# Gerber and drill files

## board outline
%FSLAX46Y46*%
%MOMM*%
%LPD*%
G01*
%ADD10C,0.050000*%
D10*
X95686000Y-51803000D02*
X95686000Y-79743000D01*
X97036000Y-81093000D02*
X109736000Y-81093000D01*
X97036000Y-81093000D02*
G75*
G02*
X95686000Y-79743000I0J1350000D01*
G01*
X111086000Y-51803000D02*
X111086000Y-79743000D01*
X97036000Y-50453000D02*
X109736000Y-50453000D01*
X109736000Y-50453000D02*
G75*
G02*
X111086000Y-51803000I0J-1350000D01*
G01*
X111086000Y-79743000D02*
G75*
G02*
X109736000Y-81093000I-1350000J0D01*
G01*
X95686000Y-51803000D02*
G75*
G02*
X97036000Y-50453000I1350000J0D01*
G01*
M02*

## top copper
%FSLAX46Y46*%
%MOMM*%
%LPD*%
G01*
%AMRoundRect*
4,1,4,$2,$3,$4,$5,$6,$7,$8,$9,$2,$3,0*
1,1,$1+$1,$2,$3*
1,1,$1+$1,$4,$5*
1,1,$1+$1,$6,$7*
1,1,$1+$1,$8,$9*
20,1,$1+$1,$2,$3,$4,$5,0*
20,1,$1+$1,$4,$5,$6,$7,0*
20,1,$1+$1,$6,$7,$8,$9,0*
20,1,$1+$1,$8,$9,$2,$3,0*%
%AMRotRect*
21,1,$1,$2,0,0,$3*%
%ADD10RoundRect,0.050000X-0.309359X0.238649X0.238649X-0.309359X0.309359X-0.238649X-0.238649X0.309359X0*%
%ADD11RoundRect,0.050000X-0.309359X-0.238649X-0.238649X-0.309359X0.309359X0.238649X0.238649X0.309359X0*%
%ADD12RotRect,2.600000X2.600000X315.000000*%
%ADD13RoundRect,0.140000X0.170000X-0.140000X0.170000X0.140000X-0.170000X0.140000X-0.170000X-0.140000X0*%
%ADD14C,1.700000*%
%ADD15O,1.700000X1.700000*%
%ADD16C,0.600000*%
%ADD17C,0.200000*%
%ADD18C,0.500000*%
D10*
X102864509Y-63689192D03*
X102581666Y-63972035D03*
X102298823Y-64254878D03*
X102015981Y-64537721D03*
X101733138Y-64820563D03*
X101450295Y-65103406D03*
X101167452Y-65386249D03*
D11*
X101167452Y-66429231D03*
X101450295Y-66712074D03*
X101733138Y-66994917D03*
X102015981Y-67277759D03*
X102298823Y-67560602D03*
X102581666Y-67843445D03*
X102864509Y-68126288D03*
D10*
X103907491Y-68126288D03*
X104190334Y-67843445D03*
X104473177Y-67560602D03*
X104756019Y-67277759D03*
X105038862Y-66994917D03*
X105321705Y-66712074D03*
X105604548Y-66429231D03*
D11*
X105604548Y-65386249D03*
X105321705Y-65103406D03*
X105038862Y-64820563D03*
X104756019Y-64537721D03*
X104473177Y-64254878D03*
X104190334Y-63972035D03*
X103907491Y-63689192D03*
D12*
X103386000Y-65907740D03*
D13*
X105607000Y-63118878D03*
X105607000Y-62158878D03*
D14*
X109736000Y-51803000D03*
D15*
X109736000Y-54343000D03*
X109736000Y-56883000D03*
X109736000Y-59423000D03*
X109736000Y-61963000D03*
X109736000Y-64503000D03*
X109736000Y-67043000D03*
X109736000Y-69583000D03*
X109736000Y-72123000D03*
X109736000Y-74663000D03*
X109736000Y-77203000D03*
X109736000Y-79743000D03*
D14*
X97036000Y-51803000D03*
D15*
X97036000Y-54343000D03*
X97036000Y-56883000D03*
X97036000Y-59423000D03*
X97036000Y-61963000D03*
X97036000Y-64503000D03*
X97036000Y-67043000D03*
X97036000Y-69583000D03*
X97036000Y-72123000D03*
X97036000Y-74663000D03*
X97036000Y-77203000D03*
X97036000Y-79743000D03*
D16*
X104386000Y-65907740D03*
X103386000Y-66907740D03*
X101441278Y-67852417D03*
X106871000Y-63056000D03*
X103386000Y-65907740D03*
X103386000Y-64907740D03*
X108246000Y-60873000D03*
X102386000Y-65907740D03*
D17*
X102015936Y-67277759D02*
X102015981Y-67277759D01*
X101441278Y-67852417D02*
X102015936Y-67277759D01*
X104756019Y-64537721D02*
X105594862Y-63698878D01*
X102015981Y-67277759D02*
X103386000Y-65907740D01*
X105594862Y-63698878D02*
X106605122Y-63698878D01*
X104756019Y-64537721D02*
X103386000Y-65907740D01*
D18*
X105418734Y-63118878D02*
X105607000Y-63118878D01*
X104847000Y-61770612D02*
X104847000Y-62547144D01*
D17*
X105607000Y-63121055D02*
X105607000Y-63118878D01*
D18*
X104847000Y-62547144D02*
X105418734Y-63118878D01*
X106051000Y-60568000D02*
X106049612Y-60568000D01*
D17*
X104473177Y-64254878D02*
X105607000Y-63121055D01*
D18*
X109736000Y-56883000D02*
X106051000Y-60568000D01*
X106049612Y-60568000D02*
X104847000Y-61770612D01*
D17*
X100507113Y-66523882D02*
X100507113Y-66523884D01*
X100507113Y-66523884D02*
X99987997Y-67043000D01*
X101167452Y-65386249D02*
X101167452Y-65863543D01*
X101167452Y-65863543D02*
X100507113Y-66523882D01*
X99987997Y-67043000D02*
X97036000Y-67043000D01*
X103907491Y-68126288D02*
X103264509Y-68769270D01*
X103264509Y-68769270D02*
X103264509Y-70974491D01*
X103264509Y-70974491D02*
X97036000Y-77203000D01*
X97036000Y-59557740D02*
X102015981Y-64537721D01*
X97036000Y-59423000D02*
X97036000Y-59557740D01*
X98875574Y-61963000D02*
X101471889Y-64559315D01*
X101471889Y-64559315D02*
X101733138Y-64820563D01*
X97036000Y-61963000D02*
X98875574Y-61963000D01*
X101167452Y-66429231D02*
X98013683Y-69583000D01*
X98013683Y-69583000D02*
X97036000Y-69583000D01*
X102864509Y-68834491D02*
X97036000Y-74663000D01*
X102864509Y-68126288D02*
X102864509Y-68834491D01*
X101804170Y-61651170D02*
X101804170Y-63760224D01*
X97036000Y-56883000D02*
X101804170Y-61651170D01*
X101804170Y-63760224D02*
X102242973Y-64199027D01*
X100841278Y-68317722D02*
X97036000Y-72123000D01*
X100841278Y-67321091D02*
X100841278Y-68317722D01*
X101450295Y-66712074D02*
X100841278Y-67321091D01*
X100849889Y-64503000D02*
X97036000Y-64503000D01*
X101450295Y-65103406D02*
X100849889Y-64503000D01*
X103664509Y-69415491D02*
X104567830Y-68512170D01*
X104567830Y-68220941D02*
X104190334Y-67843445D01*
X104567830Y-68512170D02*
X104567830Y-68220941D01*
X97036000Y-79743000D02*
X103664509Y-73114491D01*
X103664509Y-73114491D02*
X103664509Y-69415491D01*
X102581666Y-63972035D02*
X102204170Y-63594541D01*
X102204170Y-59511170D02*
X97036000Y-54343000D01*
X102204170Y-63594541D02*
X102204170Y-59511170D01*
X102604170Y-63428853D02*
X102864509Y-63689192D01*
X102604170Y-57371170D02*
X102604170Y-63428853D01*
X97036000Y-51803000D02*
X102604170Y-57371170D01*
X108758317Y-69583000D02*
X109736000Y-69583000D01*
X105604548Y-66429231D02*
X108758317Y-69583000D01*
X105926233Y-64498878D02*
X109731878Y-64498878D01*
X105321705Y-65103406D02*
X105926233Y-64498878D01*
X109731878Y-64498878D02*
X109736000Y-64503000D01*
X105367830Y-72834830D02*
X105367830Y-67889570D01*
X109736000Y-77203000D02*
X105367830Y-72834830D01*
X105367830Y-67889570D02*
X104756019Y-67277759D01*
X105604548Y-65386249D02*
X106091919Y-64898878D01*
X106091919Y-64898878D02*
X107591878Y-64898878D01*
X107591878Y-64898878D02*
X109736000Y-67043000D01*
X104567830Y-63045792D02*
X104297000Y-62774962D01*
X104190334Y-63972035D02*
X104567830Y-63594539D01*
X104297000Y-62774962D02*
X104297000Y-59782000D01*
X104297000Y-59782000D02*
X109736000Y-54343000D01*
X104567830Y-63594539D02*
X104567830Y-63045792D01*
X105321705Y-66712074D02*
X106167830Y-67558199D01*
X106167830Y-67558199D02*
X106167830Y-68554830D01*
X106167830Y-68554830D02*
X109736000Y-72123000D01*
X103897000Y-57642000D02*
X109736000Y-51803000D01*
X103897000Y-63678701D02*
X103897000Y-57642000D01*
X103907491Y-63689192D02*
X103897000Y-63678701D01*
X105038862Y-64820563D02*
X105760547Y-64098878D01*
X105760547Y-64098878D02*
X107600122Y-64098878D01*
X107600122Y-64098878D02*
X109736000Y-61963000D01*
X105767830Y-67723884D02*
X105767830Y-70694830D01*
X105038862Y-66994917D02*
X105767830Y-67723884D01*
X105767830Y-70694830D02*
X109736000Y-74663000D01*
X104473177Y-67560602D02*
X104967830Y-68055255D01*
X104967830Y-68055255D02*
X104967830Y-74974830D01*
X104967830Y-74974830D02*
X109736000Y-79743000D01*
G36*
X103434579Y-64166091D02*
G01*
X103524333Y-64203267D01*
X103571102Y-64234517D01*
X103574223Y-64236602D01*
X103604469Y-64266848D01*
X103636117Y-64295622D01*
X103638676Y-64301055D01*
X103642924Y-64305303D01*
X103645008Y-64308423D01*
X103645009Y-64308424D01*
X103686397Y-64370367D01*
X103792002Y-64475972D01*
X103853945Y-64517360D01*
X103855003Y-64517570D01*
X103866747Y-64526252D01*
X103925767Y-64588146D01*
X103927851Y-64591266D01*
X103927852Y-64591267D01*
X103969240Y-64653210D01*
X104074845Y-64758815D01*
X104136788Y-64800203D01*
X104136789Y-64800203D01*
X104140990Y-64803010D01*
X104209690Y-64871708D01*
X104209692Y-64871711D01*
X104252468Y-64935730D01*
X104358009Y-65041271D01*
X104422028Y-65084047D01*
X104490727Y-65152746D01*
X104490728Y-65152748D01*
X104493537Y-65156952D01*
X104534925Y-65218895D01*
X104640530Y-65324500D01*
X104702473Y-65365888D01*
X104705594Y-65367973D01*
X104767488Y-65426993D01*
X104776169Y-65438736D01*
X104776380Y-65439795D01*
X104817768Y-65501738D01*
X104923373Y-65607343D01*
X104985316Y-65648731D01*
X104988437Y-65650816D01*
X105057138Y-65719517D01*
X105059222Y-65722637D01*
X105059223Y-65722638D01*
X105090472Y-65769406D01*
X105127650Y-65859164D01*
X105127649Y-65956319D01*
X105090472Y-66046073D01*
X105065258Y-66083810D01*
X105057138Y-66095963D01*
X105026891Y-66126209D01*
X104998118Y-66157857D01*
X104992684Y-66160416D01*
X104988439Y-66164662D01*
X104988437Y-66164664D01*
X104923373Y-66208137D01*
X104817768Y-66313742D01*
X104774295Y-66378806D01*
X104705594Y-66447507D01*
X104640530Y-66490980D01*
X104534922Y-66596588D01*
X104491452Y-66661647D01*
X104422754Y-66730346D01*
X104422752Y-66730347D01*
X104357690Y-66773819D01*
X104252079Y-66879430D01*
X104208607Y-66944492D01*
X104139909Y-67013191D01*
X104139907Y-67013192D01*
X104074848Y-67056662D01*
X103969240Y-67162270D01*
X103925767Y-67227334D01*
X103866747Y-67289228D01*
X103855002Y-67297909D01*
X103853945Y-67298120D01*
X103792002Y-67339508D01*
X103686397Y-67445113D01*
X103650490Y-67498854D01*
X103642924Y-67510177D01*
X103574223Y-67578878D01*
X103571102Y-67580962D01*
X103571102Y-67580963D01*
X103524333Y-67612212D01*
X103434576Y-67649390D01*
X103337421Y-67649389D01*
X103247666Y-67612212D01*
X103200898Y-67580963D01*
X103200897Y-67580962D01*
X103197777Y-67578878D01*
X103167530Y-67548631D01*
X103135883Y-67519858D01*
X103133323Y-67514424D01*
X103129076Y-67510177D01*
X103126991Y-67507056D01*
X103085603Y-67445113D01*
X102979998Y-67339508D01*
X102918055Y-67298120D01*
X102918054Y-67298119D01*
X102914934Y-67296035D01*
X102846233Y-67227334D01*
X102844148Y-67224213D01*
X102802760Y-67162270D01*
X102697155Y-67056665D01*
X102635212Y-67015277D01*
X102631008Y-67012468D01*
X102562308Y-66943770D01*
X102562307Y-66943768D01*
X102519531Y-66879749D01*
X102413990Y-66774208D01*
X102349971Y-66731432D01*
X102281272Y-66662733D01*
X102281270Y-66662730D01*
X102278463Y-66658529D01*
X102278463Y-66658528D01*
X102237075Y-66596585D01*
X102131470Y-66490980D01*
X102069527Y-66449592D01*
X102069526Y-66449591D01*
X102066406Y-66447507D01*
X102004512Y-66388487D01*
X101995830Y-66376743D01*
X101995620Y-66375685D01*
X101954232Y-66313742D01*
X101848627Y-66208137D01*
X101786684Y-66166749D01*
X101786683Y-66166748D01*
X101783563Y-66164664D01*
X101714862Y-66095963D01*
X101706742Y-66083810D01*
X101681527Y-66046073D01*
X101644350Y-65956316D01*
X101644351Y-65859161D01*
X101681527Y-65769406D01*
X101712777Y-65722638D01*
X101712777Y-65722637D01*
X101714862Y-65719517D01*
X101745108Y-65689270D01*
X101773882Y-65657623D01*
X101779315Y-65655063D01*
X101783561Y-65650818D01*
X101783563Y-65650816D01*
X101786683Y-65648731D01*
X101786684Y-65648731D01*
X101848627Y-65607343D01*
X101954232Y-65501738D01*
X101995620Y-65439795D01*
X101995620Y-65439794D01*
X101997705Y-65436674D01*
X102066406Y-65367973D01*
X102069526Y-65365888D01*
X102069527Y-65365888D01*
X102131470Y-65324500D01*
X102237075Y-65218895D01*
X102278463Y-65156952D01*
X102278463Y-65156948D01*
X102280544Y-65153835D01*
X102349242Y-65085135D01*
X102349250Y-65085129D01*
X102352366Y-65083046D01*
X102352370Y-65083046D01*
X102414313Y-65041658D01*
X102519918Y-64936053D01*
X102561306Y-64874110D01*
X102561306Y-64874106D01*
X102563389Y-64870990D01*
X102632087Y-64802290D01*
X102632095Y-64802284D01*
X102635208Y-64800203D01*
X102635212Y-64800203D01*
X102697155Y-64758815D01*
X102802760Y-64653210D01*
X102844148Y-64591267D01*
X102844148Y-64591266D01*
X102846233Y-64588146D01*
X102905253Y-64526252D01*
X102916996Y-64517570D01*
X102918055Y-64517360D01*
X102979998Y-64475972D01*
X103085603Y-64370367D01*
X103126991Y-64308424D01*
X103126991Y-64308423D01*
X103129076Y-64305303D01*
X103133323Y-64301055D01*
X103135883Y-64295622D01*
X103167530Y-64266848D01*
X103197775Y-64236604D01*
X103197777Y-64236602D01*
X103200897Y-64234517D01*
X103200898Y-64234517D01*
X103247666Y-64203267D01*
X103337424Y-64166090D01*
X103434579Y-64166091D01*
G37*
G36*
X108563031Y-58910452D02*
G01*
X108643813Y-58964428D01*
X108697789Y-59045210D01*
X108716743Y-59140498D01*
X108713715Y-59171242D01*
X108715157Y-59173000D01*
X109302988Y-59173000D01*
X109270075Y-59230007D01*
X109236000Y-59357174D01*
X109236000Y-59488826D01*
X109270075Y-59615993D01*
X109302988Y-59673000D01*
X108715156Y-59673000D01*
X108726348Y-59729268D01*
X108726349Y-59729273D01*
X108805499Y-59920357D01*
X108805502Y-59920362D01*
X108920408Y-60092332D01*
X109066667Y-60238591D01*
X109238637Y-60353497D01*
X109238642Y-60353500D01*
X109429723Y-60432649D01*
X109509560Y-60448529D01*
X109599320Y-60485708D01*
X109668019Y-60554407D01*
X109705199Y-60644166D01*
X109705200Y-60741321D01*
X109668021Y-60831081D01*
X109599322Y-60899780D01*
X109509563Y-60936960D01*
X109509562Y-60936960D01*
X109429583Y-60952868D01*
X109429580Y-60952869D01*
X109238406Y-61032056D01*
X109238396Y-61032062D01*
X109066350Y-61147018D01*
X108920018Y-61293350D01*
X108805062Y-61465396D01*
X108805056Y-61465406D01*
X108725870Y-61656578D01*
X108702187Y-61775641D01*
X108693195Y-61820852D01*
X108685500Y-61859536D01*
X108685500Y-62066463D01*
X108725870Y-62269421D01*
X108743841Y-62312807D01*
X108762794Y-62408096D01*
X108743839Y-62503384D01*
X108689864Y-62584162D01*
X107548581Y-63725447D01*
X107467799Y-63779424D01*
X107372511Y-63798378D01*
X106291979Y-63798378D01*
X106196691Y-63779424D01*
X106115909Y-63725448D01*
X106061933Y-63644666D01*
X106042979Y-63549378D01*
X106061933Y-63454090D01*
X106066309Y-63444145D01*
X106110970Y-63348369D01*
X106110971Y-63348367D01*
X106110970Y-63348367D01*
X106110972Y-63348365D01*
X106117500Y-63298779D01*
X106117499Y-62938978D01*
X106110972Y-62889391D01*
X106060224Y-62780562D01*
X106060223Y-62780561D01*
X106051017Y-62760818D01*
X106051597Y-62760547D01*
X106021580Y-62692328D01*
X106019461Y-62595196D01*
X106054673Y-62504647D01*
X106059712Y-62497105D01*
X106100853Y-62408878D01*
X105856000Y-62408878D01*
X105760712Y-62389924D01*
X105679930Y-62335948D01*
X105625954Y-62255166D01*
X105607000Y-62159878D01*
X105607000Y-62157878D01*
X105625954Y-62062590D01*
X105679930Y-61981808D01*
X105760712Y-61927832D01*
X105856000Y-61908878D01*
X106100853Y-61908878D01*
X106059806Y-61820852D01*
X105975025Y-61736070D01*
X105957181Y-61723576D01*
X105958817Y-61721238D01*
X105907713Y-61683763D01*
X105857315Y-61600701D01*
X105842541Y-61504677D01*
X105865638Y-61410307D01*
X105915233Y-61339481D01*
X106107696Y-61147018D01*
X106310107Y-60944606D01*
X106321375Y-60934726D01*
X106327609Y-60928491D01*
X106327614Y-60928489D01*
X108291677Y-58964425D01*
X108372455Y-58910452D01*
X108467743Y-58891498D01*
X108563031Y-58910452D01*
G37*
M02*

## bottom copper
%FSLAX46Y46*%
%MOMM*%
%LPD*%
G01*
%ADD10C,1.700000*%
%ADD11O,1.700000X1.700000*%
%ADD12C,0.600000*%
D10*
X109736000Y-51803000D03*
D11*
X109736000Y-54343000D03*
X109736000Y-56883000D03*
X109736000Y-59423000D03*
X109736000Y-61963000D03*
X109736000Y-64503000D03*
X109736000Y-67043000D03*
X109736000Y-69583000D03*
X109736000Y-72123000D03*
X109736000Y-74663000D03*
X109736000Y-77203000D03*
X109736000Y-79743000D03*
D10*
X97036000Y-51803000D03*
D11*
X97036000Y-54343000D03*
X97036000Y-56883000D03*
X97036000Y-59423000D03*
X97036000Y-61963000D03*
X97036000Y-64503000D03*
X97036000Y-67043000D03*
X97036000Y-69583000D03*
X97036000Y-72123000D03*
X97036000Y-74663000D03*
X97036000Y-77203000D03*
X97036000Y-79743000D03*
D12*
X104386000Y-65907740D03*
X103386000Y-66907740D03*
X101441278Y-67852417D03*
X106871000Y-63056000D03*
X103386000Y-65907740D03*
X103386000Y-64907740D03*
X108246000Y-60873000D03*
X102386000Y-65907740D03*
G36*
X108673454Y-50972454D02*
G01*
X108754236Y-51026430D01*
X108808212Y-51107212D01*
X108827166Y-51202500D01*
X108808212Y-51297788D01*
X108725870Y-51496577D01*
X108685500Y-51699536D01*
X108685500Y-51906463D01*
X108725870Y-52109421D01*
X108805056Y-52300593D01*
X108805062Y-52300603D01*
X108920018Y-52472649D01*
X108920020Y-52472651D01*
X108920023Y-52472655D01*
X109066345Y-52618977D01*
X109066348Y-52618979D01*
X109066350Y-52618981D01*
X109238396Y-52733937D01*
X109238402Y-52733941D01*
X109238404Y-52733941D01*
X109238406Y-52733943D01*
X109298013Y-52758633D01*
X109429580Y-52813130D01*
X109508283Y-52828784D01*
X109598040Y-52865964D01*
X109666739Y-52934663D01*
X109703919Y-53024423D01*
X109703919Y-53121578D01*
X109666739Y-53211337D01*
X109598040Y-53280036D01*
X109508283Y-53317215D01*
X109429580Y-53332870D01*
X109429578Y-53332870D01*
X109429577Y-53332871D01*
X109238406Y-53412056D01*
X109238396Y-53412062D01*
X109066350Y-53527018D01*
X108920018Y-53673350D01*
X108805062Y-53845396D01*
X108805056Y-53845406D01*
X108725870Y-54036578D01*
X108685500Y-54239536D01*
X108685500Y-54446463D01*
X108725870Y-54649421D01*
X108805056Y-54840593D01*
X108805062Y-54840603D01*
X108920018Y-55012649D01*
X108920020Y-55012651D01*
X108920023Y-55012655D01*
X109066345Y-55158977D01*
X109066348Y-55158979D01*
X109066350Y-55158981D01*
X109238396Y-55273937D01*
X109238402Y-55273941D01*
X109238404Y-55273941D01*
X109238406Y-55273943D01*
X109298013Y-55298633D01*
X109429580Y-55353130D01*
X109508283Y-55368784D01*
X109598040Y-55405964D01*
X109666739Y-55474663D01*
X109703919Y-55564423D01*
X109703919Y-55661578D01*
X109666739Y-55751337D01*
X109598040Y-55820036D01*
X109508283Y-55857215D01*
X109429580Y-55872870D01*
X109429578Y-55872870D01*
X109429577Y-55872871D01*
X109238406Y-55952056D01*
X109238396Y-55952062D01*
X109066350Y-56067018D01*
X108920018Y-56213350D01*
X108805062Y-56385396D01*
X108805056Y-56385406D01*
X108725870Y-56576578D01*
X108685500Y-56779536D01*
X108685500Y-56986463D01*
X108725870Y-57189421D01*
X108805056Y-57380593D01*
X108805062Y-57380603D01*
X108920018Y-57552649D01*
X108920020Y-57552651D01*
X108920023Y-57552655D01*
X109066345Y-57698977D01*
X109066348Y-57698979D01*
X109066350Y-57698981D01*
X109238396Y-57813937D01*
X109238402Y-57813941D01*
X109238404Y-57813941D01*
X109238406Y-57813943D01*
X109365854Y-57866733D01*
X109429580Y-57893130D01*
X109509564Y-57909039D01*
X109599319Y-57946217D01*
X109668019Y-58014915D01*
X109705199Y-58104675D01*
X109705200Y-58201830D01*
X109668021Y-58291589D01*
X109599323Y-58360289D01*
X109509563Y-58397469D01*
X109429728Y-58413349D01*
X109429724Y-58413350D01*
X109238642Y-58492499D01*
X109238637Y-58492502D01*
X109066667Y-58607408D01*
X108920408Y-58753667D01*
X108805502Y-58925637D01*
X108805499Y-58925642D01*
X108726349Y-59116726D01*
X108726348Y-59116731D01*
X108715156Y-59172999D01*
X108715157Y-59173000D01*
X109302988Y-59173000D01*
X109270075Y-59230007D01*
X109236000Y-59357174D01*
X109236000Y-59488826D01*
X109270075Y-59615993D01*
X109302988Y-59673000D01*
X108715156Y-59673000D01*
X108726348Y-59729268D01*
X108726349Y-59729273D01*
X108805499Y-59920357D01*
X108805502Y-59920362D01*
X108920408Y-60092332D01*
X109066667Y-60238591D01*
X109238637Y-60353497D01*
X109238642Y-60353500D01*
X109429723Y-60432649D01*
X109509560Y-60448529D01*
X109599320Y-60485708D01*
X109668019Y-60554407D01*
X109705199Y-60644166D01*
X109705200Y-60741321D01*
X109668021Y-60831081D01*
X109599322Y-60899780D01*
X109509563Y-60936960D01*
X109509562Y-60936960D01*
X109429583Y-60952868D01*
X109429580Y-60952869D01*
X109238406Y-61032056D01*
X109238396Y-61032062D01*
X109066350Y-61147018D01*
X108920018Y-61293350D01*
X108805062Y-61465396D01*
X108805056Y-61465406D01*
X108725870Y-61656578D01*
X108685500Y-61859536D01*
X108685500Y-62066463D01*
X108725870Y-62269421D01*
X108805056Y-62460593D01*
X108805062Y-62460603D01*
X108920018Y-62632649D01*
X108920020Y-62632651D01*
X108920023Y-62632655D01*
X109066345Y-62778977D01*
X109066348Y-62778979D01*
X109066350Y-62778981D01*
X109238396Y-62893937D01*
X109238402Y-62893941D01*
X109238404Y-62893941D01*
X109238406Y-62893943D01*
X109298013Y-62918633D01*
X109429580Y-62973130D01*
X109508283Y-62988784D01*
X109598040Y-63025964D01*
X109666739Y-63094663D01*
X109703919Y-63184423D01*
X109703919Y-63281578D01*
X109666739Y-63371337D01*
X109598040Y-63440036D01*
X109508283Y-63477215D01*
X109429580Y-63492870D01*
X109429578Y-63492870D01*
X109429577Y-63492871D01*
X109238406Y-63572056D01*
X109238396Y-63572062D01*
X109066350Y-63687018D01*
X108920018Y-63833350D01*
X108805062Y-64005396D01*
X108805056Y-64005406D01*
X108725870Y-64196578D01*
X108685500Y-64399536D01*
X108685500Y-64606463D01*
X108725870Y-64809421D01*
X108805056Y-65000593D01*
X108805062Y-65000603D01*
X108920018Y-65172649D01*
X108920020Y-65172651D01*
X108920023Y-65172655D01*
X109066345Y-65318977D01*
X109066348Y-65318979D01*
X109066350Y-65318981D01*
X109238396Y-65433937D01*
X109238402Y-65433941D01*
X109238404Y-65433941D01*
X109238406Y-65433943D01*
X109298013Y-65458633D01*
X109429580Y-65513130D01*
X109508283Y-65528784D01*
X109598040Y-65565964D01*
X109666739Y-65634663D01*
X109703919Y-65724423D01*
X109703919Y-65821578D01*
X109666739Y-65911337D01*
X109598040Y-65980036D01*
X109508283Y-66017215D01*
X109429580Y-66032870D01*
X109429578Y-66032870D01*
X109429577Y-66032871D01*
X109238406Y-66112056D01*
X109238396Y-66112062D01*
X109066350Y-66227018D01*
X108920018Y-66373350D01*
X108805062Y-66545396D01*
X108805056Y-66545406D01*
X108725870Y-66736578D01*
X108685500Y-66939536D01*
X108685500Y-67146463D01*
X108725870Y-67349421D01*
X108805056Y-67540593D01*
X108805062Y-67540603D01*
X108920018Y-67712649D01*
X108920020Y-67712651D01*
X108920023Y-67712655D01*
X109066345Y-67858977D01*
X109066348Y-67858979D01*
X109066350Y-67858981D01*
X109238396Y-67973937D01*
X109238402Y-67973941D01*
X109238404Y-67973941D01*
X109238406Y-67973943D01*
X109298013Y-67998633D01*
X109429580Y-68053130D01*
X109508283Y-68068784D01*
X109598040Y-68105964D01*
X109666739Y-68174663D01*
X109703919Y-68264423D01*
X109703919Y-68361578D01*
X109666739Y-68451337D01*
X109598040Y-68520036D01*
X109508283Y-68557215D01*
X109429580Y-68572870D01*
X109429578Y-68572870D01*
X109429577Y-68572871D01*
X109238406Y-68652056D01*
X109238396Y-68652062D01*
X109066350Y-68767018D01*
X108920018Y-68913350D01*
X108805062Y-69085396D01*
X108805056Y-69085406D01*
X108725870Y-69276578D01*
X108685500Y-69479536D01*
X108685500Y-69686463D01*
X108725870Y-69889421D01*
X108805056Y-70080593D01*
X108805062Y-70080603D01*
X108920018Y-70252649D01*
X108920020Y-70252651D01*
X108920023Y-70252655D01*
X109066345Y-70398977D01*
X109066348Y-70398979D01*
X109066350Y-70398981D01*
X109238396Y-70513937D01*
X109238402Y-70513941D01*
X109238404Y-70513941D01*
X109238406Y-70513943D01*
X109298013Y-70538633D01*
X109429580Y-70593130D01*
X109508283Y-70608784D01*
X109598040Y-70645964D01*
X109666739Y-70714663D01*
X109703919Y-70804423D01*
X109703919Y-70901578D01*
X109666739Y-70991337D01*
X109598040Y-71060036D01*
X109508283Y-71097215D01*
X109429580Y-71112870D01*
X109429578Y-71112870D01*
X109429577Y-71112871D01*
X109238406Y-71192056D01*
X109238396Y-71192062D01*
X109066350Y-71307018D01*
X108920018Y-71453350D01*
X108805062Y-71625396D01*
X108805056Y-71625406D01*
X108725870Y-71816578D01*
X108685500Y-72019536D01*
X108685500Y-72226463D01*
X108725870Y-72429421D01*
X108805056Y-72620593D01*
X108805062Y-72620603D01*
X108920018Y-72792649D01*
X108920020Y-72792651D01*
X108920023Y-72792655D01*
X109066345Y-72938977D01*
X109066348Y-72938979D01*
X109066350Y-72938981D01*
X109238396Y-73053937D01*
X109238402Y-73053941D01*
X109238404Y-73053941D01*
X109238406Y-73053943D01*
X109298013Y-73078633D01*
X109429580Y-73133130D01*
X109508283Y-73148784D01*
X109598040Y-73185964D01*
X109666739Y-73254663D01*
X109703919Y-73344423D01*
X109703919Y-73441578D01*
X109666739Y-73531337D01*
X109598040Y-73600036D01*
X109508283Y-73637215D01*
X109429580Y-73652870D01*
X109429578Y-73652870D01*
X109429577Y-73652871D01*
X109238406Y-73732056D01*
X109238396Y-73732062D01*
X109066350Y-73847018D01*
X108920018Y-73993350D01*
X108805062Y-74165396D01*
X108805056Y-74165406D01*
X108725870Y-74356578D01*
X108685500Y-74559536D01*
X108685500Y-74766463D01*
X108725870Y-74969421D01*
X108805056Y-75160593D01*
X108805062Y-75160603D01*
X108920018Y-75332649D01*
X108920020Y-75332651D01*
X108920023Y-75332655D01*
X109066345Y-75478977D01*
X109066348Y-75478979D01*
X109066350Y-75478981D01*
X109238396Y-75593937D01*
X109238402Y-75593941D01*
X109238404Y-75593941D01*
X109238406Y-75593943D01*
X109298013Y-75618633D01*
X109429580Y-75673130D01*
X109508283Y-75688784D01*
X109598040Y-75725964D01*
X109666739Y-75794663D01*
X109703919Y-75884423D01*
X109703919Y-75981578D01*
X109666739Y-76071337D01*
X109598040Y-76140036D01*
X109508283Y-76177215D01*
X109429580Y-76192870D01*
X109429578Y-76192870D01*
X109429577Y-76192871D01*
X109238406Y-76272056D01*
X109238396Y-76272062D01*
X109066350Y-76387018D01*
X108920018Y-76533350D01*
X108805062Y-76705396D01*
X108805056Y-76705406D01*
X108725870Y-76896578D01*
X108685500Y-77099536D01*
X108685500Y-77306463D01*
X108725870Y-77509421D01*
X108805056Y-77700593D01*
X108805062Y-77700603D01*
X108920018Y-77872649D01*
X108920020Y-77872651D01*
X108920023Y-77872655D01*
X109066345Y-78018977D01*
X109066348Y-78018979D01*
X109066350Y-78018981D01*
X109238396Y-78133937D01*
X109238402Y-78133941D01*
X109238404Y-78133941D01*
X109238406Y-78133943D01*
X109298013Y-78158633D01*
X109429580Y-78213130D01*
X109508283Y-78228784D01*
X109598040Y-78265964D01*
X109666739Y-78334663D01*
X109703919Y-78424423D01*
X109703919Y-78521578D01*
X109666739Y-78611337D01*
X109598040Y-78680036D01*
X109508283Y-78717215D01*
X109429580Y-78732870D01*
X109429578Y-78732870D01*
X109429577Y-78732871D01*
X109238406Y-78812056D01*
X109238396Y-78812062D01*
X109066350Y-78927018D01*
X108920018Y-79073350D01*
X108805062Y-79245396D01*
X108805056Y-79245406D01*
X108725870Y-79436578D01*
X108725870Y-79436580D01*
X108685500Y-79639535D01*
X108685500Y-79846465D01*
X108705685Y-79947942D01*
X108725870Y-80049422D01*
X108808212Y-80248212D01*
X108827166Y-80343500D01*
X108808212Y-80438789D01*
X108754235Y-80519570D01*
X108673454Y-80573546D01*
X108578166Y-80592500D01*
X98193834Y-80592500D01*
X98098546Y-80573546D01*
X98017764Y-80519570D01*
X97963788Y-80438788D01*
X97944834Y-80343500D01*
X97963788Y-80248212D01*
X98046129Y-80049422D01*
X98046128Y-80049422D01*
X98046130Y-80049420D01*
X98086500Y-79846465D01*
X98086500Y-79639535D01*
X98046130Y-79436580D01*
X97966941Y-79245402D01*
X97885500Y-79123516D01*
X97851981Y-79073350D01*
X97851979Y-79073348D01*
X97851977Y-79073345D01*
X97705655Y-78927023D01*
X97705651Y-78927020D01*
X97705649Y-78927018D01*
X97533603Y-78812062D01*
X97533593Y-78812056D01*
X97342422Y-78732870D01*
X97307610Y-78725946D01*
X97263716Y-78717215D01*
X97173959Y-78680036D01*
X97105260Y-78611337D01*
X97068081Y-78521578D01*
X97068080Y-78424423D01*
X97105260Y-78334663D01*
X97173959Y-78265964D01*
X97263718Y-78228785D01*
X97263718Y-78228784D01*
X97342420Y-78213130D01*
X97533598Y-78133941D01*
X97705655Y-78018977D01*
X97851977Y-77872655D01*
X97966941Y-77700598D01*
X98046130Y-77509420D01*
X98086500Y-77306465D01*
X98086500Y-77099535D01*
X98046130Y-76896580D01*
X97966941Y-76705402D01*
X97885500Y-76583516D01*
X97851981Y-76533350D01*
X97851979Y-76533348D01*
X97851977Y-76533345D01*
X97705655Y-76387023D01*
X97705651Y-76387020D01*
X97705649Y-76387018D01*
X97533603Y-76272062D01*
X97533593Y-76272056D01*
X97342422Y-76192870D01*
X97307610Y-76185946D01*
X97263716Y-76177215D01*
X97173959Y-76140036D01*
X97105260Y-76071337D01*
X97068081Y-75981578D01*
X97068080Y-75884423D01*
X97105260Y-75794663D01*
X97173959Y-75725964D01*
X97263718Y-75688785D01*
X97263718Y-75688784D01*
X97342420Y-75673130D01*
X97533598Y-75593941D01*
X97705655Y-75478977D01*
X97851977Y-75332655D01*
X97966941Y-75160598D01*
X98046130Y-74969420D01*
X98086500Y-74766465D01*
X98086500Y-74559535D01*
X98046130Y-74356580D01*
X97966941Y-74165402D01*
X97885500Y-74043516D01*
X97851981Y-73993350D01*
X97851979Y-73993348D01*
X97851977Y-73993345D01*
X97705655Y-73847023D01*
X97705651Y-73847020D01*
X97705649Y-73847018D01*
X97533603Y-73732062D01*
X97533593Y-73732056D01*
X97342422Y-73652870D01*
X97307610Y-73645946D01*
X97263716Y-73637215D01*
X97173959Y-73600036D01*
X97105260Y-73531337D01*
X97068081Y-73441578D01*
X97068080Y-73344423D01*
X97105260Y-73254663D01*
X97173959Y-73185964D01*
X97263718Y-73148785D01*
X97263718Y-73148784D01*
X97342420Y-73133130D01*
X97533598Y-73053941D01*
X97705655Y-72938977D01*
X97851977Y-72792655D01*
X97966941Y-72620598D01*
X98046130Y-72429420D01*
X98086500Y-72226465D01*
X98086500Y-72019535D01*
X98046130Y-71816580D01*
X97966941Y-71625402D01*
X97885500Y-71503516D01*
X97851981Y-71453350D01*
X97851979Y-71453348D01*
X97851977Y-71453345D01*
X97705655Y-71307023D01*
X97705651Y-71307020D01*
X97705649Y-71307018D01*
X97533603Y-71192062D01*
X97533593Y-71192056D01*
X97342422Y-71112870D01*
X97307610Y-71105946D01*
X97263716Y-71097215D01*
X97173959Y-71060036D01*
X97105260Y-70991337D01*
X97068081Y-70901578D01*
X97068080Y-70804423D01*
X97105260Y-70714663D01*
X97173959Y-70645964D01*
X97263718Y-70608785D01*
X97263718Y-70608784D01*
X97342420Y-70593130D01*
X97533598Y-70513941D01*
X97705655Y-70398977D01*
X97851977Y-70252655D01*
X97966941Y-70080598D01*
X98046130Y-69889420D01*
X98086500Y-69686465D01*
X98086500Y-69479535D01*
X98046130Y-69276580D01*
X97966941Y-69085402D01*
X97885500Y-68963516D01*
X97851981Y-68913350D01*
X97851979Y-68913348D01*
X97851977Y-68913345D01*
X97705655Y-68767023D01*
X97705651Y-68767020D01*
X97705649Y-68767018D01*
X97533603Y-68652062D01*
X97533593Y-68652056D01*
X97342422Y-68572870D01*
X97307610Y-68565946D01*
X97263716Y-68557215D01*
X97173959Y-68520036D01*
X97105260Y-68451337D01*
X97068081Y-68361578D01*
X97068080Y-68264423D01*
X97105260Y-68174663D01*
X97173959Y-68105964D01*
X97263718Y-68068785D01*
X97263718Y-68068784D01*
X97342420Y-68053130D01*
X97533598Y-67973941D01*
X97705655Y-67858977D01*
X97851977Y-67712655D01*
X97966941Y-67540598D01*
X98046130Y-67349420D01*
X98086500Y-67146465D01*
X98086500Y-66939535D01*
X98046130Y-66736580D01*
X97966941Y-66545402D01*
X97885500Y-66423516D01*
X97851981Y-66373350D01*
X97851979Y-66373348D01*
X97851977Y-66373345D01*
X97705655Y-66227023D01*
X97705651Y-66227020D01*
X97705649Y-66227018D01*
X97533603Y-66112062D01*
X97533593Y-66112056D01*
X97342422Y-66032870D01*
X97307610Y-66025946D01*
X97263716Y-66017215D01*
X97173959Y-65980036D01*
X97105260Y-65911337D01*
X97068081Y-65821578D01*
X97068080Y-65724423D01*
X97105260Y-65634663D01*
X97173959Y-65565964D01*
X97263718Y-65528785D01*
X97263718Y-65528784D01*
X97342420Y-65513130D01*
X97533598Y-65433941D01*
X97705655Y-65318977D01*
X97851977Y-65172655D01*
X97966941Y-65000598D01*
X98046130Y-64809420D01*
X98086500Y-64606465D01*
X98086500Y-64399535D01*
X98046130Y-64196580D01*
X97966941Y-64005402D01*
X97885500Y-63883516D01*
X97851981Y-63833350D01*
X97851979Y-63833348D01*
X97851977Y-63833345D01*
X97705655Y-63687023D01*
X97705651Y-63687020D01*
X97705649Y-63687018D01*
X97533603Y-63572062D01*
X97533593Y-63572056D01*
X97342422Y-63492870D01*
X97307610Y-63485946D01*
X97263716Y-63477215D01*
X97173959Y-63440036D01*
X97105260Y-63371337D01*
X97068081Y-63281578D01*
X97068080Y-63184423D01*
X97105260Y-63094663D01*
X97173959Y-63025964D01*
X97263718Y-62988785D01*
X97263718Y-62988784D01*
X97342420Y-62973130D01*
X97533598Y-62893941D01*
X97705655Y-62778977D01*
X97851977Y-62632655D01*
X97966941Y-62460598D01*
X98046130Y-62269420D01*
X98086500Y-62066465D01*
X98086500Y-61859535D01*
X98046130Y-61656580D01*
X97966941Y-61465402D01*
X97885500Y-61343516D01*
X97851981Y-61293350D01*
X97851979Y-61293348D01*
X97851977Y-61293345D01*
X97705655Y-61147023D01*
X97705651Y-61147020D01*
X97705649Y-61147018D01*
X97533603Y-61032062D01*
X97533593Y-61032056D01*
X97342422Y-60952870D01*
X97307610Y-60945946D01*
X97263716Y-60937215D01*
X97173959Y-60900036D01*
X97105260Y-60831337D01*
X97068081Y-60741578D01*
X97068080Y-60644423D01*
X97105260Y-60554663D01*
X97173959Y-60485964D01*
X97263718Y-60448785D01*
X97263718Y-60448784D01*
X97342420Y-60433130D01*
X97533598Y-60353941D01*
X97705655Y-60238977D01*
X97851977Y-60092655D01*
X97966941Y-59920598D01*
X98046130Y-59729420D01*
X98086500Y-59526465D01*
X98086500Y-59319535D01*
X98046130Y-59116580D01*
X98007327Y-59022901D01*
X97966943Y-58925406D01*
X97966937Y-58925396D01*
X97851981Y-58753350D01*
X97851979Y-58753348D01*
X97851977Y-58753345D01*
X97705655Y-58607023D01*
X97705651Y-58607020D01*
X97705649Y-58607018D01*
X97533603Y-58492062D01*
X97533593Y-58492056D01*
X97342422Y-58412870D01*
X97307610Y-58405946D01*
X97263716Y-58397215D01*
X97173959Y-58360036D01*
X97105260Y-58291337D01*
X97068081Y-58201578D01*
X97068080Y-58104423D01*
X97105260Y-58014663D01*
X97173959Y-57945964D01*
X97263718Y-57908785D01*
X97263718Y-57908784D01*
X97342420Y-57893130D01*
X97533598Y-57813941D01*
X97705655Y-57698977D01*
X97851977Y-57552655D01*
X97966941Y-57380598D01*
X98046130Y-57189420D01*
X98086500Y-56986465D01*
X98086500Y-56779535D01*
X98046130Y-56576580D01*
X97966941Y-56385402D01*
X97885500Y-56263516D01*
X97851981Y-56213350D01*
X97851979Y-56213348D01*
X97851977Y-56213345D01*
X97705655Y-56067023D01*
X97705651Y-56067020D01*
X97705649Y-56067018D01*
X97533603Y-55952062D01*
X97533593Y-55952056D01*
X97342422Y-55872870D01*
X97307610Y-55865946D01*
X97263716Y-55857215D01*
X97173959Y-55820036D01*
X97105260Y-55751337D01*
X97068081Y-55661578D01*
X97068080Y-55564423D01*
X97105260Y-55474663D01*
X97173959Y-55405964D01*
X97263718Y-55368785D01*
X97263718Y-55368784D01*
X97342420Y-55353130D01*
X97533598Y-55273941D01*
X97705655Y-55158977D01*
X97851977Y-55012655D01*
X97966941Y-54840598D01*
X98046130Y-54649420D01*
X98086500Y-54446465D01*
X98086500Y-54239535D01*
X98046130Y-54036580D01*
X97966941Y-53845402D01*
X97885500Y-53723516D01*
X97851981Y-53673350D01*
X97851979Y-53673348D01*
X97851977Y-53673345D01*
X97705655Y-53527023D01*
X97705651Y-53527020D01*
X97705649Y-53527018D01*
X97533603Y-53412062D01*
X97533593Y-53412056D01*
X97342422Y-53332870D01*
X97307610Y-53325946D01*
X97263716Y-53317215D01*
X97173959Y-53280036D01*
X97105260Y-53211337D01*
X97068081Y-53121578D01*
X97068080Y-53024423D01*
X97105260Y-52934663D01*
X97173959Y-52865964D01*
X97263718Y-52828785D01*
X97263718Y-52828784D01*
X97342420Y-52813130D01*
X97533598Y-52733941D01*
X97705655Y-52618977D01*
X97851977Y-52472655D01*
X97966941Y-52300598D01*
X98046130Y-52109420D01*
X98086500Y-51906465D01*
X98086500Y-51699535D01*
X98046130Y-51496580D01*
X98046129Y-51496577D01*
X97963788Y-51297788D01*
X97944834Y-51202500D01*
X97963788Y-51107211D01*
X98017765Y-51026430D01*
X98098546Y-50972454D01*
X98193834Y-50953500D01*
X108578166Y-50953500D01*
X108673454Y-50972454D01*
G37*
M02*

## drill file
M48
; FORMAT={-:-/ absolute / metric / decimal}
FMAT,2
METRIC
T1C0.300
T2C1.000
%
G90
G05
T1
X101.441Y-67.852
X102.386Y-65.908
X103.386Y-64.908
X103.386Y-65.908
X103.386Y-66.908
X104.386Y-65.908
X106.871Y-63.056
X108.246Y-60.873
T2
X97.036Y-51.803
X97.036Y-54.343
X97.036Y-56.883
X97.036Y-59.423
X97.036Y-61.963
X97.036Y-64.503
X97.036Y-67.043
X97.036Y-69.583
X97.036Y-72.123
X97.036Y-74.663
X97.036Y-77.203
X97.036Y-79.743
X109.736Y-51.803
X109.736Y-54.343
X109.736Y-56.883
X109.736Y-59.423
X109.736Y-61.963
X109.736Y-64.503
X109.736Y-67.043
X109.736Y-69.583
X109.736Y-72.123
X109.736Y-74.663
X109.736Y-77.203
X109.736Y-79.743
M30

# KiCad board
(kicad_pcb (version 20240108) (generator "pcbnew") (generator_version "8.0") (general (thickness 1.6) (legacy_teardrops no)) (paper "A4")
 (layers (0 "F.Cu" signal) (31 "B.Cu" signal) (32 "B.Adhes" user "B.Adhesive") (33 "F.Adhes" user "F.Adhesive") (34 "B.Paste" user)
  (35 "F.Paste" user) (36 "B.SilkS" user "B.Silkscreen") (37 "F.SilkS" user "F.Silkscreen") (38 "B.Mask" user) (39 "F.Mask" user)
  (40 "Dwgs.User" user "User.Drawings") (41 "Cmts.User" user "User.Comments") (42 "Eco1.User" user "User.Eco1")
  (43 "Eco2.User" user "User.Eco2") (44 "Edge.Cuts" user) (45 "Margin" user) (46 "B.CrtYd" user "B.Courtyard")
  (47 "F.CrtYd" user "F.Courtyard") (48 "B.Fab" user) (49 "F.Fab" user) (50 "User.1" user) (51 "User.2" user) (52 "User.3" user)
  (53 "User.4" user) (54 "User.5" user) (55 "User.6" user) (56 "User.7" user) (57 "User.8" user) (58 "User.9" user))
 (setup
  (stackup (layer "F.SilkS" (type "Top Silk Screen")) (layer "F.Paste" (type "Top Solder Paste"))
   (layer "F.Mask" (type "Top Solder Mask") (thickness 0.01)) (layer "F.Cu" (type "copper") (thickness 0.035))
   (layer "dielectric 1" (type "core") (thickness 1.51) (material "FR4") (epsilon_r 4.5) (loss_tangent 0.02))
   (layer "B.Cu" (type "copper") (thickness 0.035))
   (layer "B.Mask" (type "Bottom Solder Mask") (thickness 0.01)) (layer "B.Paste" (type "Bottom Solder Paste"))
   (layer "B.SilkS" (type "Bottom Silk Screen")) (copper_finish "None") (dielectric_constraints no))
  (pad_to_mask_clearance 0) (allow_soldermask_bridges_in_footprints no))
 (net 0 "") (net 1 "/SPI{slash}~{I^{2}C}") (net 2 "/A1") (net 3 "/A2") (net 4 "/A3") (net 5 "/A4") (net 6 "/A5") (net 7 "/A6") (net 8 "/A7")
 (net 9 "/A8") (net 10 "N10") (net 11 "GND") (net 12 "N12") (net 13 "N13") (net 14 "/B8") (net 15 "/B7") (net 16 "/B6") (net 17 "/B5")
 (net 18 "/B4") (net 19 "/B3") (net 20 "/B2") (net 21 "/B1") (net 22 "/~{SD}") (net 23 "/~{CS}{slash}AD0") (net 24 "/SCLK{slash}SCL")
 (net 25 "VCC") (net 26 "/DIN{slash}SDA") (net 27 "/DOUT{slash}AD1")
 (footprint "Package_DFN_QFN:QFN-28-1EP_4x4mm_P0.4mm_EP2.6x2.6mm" (layer "F.Cu") (at 103.386 65.90774 -45)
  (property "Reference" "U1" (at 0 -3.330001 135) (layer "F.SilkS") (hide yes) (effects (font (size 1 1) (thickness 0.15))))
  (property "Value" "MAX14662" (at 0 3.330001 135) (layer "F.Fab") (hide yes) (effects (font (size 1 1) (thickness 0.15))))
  (pad "" smd roundrect (at -0.65 -0.65 315) (size 1.05 1.05) (layers "F.Paste") (roundrect_rratio 0.238095))
  (pad "" smd roundrect (at -0.65 0.65 315) (size 1.05 1.05) (layers "F.Paste") (roundrect_rratio 0.238095))
  (pad "" smd roundrect (at 0.65 -0.65 315) (size 1.05 1.05) (layers "F.Paste") (roundrect_rratio 0.238095))
  (pad "" smd roundrect (at 0.65 0.65 315) (size 1.05 1.05) (layers "F.Paste") (roundrect_rratio 0.238095))
  (pad "1" smd roundrect (at -1.9375 -1.200001 315) (size 0.875 0.2) (layers "F.Cu" "F.Paste" "F.Mask") (roundrect_rratio 0.25)
   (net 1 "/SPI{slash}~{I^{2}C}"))
  (pad "2" smd roundrect (at -1.9375 -0.8 315) (size 0.875 0.2) (layers "F.Cu" "F.Paste" "F.Mask") (roundrect_rratio 0.25) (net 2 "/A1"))
  (pad "3" smd roundrect (at -1.9375 -0.4 315) (size 0.875 0.2) (layers "F.Cu" "F.Paste" "F.Mask") (roundrect_rratio 0.25) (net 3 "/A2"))
  (pad "4" smd roundrect (at -1.937499 0 315) (size 0.875 0.2) (layers "F.Cu" "F.Paste" "F.Mask") (roundrect_rratio 0.25) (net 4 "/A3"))
  (pad "5" smd roundrect (at -1.9375 0.4 315) (size 0.875 0.2) (layers "F.Cu" "F.Paste" "F.Mask") (roundrect_rratio 0.25) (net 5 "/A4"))
  (pad "6" smd roundrect (at -1.9375 0.8 315) (size 0.875 0.2) (layers "F.Cu" "F.Paste" "F.Mask") (roundrect_rratio 0.25) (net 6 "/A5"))
  (pad "7" smd roundrect (at -1.9375 1.200001 315) (size 0.875 0.2) (layers "F.Cu" "F.Paste" "F.Mask") (roundrect_rratio 0.25) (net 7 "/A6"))
  (pad "8" smd roundrect (at -1.200001 1.9375 315) (size 0.2 0.875) (layers "F.Cu" "F.Paste" "F.Mask") (roundrect_rratio 0.25) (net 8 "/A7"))
  (pad "9" smd roundrect (at -0.8 1.9375 315) (size 0.2 0.875) (layers "F.Cu" "F.Paste" "F.Mask") (roundrect_rratio 0.25) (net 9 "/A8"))
  (pad "10" smd roundrect (at -0.4 1.9375 315) (size 0.2 0.875) (layers "F.Cu" "F.Paste" "F.Mask") (roundrect_rratio 0.25) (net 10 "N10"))
  (pad "11" smd roundrect (at 0 1.937499 315) (size 0.2 0.875) (layers "F.Cu" "F.Paste" "F.Mask") (roundrect_rratio 0.25) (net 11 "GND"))
  (pad "12" smd roundrect (at 0.4 1.9375 315) (size 0.2 0.875) (layers "F.Cu" "F.Paste" "F.Mask") (roundrect_rratio 0.25) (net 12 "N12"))
  (pad "13" smd roundrect (at 0.8 1.9375 315) (size 0.2 0.875) (layers "F.Cu" "F.Paste" "F.Mask") (roundrect_rratio 0.25) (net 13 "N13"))
  (pad "14" smd roundrect (at 1.200001 1.9375 315) (size 0.2 0.875) (layers "F.Cu" "F.Paste" "F.Mask") (roundrect_rratio 0.25)
   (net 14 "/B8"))
  (pad "15" smd roundrect (at 1.9375 1.200001 315) (size 0.875 0.2) (layers "F.Cu" "F.Paste" "F.Mask") (roundrect_rratio 0.25)
   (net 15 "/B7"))
  (pad "16" smd roundrect (at 1.9375 0.8 315) (size 0.875 0.2) (layers "F.Cu" "F.Paste" "F.Mask") (roundrect_rratio 0.25) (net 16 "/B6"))
  (pad "17" smd roundrect (at 1.9375 0.4 315) (size 0.875 0.2) (layers "F.Cu" "F.Paste" "F.Mask") (roundrect_rratio 0.25) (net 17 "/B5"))
  (pad "18" smd roundrect (at 1.937499 0 315) (size 0.875 0.2) (layers "F.Cu" "F.Paste" "F.Mask") (roundrect_rratio 0.25) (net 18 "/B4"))
  (pad "19" smd roundrect (at 1.9375 -0.4 315) (size 0.875 0.2) (layers "F.Cu" "F.Paste" "F.Mask") (roundrect_rratio 0.25) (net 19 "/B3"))
  (pad "20" smd roundrect (at 1.9375 -0.8 315) (size 0.875 0.2) (layers "F.Cu" "F.Paste" "F.Mask") (roundrect_rratio 0.25) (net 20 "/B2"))
  (pad "21" smd roundrect (at 1.9375 -1.200001 315) (size 0.875 0.2) (layers "F.Cu" "F.Paste" "F.Mask") (roundrect_rratio 0.25)
   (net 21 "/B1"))
  (pad "22" smd roundrect (at 1.200001 -1.9375 315) (size 0.2 0.875) (layers "F.Cu" "F.Paste" "F.Mask") (roundrect_rratio 0.25)
   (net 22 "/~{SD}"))
  (pad "23" smd roundrect (at 0.8 -1.9375 315) (size 0.2 0.875) (layers "F.Cu" "F.Paste" "F.Mask") (roundrect_rratio 0.25)
   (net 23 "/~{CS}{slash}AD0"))
  (pad "24" smd roundrect (at 0.4 -1.9375 315) (size 0.2 0.875) (layers "F.Cu" "F.Paste" "F.Mask") (roundrect_rratio 0.25)
   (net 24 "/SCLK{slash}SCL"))
  (pad "25" smd roundrect (at 0 -1.937499 315) (size 0.2 0.875) (layers "F.Cu" "F.Paste" "F.Mask") (roundrect_rratio 0.25) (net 11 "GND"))
  (pad "26" smd roundrect (at -0.4 -1.9375 315) (size 0.2 0.875) (layers "F.Cu" "F.Paste" "F.Mask") (roundrect_rratio 0.25) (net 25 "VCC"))
  (pad "27" smd roundrect (at -0.8 -1.9375 315) (size 0.2 0.875) (layers "F.Cu" "F.Paste" "F.Mask") (roundrect_rratio 0.25)
   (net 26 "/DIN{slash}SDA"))
  (pad "28" smd roundrect (at -1.200001 -1.9375 315) (size 0.2 0.875) (layers "F.Cu" "F.Paste" "F.Mask") (roundrect_rratio 0.25)
   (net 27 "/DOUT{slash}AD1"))
  (pad "29" smd rect (at 0 0 315) (size 2.6 2.6) (layers "F.Cu" "F.Mask") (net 11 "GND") (zone_connect 2)))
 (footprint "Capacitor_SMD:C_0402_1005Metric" (layer "F.Cu") (at 105.607 62.638878 90)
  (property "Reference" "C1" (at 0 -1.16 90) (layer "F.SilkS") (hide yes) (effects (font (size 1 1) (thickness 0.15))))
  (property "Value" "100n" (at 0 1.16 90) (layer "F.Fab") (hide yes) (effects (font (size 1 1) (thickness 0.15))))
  (pad "1" smd roundrect (at -0.48 0 90) (size 0.56 0.62) (layers "F.Cu" "F.Paste" "F.Mask") (roundrect_rratio 0.25) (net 25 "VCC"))
  (pad "2" smd roundrect (at 0.48 0 90) (size 0.56 0.62) (layers "F.Cu" "F.Paste" "F.Mask") (roundrect_rratio 0.25) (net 11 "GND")))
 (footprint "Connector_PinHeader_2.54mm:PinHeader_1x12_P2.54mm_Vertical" (layer "B.Cu") (at 109.736 51.803 180)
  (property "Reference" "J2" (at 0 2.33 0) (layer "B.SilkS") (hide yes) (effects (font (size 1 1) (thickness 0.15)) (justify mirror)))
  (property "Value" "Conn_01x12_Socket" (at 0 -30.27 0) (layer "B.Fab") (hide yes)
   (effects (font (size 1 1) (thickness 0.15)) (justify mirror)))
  (pad "1" thru_hole circle (at 0 0 180) (size 1.7 1.7) (drill 1) (layers "*.Cu" "*.Mask") (remove_unused_layers no)
   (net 27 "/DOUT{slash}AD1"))
  (pad "2" thru_hole oval (at 0 -2.54 180) (size 1.7 1.7) (drill 1) (layers "*.Cu" "*.Mask") (remove_unused_layers no)
   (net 26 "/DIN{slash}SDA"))
  (pad "3" thru_hole oval (at 0 -5.08 180) (size 1.7 1.7) (drill 1) (layers "*.Cu" "*.Mask") (remove_unused_layers no) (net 25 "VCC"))
  (pad "4" thru_hole oval (at 0 -7.62 180) (size 1.7 1.7) (drill 1) (layers "*.Cu" "*.Mask") (remove_unused_layers no) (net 11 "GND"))
  (pad "5" thru_hole oval (at 0 -10.16 180) (size 1.7 1.7) (drill 1) (layers "*.Cu" "*.Mask") (remove_unused_layers no)
   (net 24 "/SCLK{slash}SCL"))
  (pad "6" thru_hole oval (at 0 -12.7 180) (size 1.7 1.7) (drill 1) (layers "*.Cu" "*.Mask") (remove_unused_layers no)
   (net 23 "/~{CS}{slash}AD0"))
  (pad "7" thru_hole oval (at 0 -15.24 180) (size 1.7 1.7) (drill 1) (layers "*.Cu" "*.Mask") (remove_unused_layers no) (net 22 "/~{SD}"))
  (pad "8" thru_hole oval (at 0 -17.78 180) (size 1.7 1.7) (drill 1) (layers "*.Cu" "*.Mask") (remove_unused_layers no) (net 21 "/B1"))
  (pad "9" thru_hole oval (at 0 -20.32 180) (size 1.7 1.7) (drill 1) (layers "*.Cu" "*.Mask") (remove_unused_layers no) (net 20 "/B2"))
  (pad "10" thru_hole oval (at 0 -22.86 180) (size 1.7 1.7) (drill 1) (layers "*.Cu" "*.Mask") (remove_unused_layers no) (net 19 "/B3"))
  (pad "11" thru_hole oval (at 0 -25.4 180) (size 1.7 1.7) (drill 1) (layers "*.Cu" "*.Mask") (remove_unused_layers no) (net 18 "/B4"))
  (pad "12" thru_hole oval (at 0 -27.94 180) (size 1.7 1.7) (drill 1) (layers "*.Cu" "*.Mask") (remove_unused_layers no) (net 17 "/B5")))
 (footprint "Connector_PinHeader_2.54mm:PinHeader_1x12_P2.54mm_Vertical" (layer "B.Cu") (at 97.036 51.803 180)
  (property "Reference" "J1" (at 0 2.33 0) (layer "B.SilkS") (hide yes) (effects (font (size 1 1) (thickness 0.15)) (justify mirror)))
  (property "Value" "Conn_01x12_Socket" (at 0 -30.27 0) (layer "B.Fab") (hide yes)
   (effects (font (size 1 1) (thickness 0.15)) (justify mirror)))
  (pad "1" thru_hole circle (at 0 0 180) (size 1.7 1.7) (drill 1) (layers "*.Cu" "*.Mask") (remove_unused_layers no)
   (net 1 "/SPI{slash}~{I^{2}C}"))
  (pad "2" thru_hole oval (at 0 -2.54 180) (size 1.7 1.7) (drill 1) (layers "*.Cu" "*.Mask") (remove_unused_layers no) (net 2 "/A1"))
  (pad "3" thru_hole oval (at 0 -5.08 180) (size 1.7 1.7) (drill 1) (layers "*.Cu" "*.Mask") (remove_unused_layers no) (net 3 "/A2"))
  (pad "4" thru_hole oval (at 0 -7.62 180) (size 1.7 1.7) (drill 1) (layers "*.Cu" "*.Mask") (remove_unused_layers no) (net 4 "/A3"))
  (pad "5" thru_hole oval (at 0 -10.16 180) (size 1.7 1.7) (drill 1) (layers "*.Cu" "*.Mask") (remove_unused_layers no) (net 5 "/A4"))
  (pad "6" thru_hole oval (at 0 -12.7 180) (size 1.7 1.7) (drill 1) (layers "*.Cu" "*.Mask") (remove_unused_layers no) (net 6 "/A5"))
  (pad "7" thru_hole oval (at 0 -15.24 180) (size 1.7 1.7) (drill 1) (layers "*.Cu" "*.Mask") (remove_unused_layers no) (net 7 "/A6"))
  (pad "8" thru_hole oval (at 0 -17.78 180) (size 1.7 1.7) (drill 1) (layers "*.Cu" "*.Mask") (remove_unused_layers no) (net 8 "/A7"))
  (pad "9" thru_hole oval (at 0 -20.32 180) (size 1.7 1.7) (drill 1) (layers "*.Cu" "*.Mask") (remove_unused_layers no) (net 9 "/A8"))
  (pad "10" thru_hole oval (at 0 -22.86 180) (size 1.7 1.7) (drill 1) (layers "*.Cu" "*.Mask") (remove_unused_layers no) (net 14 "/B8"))
  (pad "11" thru_hole oval (at 0 -25.4 180) (size 1.7 1.7) (drill 1) (layers "*.Cu" "*.Mask") (remove_unused_layers no) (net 15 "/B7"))
  (pad "12" thru_hole oval (at 0 -27.94 180) (size 1.7 1.7) (drill 1) (layers "*.Cu" "*.Mask") (remove_unused_layers no) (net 16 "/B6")))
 (gr_line (start 95.686 51.803) (end 95.686 79.743) (stroke (width 0.05) (type default)) (layer "Edge.Cuts"))
 (gr_line (start 97.036 81.093) (end 109.736 81.093) (stroke (width 0.05) (type default)) (layer "Edge.Cuts"))
 (gr_arc (start 97.036 81.093) (mid 96.081406 80.697594) (end 95.686 79.743) (stroke (width 0.05) (type default)) (layer "Edge.Cuts"))
 (gr_line (start 111.086 51.803) (end 111.086 79.743) (stroke (width 0.05) (type default)) (layer "Edge.Cuts"))
 (gr_line (start 97.036 50.453) (end 109.736 50.453) (stroke (width 0.05) (type default)) (layer "Edge.Cuts"))
 (gr_arc (start 109.736 50.453) (mid 110.690594 50.848406) (end 111.086 51.803) (stroke (width 0.05) (type default)) (layer "Edge.Cuts"))
 (gr_arc (start 111.086 79.743) (mid 110.690594 80.697594) (end 109.736 81.093) (stroke (width 0.05) (type default)) (layer "Edge.Cuts"))
 (gr_arc (start 95.686 51.803) (mid 96.081406 50.848406) (end 97.036 50.453) (stroke (width 0.05) (type default)) (layer "Edge.Cuts"))
 (segment (start 102.015936 67.277759) (end 102.015981 67.277759) (width 0.2) (layer "F.Cu") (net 11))
 (segment (start 101.441278 67.852417) (end 102.015936 67.277759) (width 0.2) (layer "F.Cu") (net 11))
 (segment (start 104.756019 64.537721) (end 105.594862 63.698878) (width 0.2) (layer "F.Cu") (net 11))
 (segment (start 102.015981 67.277759) (end 103.386 65.90774) (width 0.2) (layer "F.Cu") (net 11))
 (segment (start 105.594862 63.698878) (end 106.605122 63.698878) (width 0.2) (layer "F.Cu") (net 11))
 (segment (start 104.756019 64.537721) (end 103.386 65.90774) (width 0.2) (layer "F.Cu") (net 11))
 (via (at 104.386 65.90774) (size 0.6) (drill 0.3) (layers "F.Cu" "B.Cu") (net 11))
 (via (at 103.386 66.90774) (size 0.6) (drill 0.3) (layers "F.Cu" "B.Cu") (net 11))
 (via (at 101.441278 67.852417) (size 0.6) (drill 0.3) (layers "F.Cu" "B.Cu") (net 11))
 (via (at 106.871 63.056) (size 0.6) (drill 0.3) (layers "F.Cu" "B.Cu") (free yes) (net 11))
 (via (at 103.386 65.90774) (size 0.6) (drill 0.3) (layers "F.Cu" "B.Cu") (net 11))
 (via (at 103.386 64.90774) (size 0.6) (drill 0.3) (layers "F.Cu" "B.Cu") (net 11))
 (via (at 108.246 60.873) (size 0.6) (drill 0.3) (layers "F.Cu" "B.Cu") (free yes) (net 11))
 (via (at 102.386 65.90774) (size 0.6) (drill 0.3) (layers "F.Cu" "B.Cu") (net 11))
 (segment (start 105.418734 63.118878) (end 105.607 63.118878) (width 0.5) (layer "F.Cu") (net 25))
 (segment (start 104.847 61.770612) (end 104.847 62.547144) (width 0.5) (layer "F.Cu") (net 25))
 (segment (start 105.607 63.121055) (end 105.607 63.118878) (width 0.2) (layer "F.Cu") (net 25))
 (segment (start 104.847 62.547144) (end 105.418734 63.118878) (width 0.5) (layer "F.Cu") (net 25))
 (segment (start 106.051 60.568) (end 106.049612 60.568) (width 0.5) (layer "F.Cu") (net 25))
 (segment (start 104.473177 64.254878) (end 105.607 63.121055) (width 0.2) (layer "F.Cu") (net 25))
 (segment (start 109.736 56.883) (end 106.051 60.568) (width 0.5) (layer "F.Cu") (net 25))
 (segment (start 106.049612 60.568) (end 104.847 61.770612) (width 0.5) (layer "F.Cu") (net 25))
 (segment (start 100.507113 66.523882) (end 100.507113 66.523884) (width 0.2) (layer "F.Cu") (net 7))
 (segment (start 100.507113 66.523884) (end 99.987997 67.043) (width 0.2) (layer "F.Cu") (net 7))
 (segment (start 101.167452 65.386249) (end 101.167452 65.863543) (width 0.2) (layer "F.Cu") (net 7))
 (segment (start 101.167452 65.863543) (end 100.507113 66.523882) (width 0.2) (layer "F.Cu") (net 7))
 (segment (start 99.987997 67.043) (end 97.036 67.043) (width 0.2) (layer "F.Cu") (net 7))
 (segment (start 103.907491 68.126288) (end 103.264509 68.76927) (width 0.2) (layer "F.Cu") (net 15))
 (segment (start 103.264509 68.76927) (end 103.264509 70.974491) (width 0.2) (layer "F.Cu") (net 15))
 (segment (start 103.264509 70.974491) (end 97.036 77.203) (width 0.2) (layer "F.Cu") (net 15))
 (segment (start 97.036 59.55774) (end 102.015981 64.537721) (width 0.2) (layer "F.Cu") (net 4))
 (segment (start 97.036 59.423) (end 97.036 59.55774) (width 0.2) (layer "F.Cu") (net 4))
 (segment (start 98.875574 61.963) (end 101.471889 64.559315) (width 0.2) (layer "F.Cu") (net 5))
 (segment (start 101.471889 64.559315) (end 101.733138 64.820563) (width 0.2) (layer "F.Cu") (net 5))
 (segment (start 97.036 61.963) (end 98.875574 61.963) (width 0.2) (layer "F.Cu") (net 5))
 (segment (start 101.167452 66.429231) (end 98.013683 69.583) (width 0.2) (layer "F.Cu") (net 8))
 (segment (start 98.013683 69.583) (end 97.036 69.583) (width 0.2) (layer "F.Cu") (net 8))
 (segment (start 102.864509 68.834491) (end 97.036 74.663) (width 0.2) (layer "F.Cu") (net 14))
 (segment (start 102.864509 68.126288) (end 102.864509 68.834491) (width 0.2) (layer "F.Cu") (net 14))
 (segment (start 101.80417 61.65117) (end 101.80417 63.760224) (width 0.2) (layer "F.Cu") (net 3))
 (segment (start 97.036 56.883) (end 101.80417 61.65117) (width 0.2) (layer "F.Cu") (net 3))
 (segment (start 101.80417 63.760224) (end 102.242973 64.199027) (width 0.2) (layer "F.Cu") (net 3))
 (segment (start 100.841278 68.317722) (end 97.036 72.123) (width 0.2) (layer "F.Cu") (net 9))
 (segment (start 100.841278 67.321091) (end 100.841278 68.317722) (width 0.2) (layer "F.Cu") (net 9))
 (segment (start 101.450295 66.712074) (end 100.841278 67.321091) (width 0.2) (layer "F.Cu") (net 9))
 (segment (start 100.849889 64.503) (end 97.036 64.503) (width 0.2) (layer "F.Cu") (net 6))
 (segment (start 101.450295 65.103406) (end 100.849889 64.503) (width 0.2) (layer "F.Cu") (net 6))
 (segment (start 103.664509 69.415491) (end 104.56783 68.51217) (width 0.2) (layer "F.Cu") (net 16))
 (segment (start 104.56783 68.220941) (end 104.190334 67.843445) (width 0.2) (layer "F.Cu") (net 16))
 (segment (start 104.56783 68.51217) (end 104.56783 68.220941) (width 0.2) (layer "F.Cu") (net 16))
 (segment (start 97.036 79.743) (end 103.664509 73.114491) (width 0.2) (layer "F.Cu") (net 16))
 (segment (start 103.664509 73.114491) (end 103.664509 69.415491) (width 0.2) (layer "F.Cu") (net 16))
 (segment (start 102.581666 63.972035) (end 102.20417 63.594541) (width 0.2) (layer "F.Cu") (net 2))
 (segment (start 102.20417 59.51117) (end 97.036 54.343) (width 0.2) (layer "F.Cu") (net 2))
 (segment (start 102.20417 63.594541) (end 102.20417 59.51117) (width 0.2) (layer "F.Cu") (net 2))
 (segment (start 102.60417 63.428853) (end 102.864509 63.689192) (width 0.2) (layer "F.Cu") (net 1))
 (segment (start 102.60417 57.37117) (end 102.60417 63.428853) (width 0.2) (layer "F.Cu") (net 1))
 (segment (start 97.036 51.803) (end 102.60417 57.37117) (width 0.2) (layer "F.Cu") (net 1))
 (segment (start 108.758317 69.583) (end 109.736 69.583) (width 0.2) (layer "F.Cu") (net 21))
 (segment (start 105.604548 66.429231) (end 108.758317 69.583) (width 0.2) (layer "F.Cu") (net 21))
 (segment (start 105.926233 64.498878) (end 109.731878 64.498878) (width 0.2) (layer "F.Cu") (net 23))
 (segment (start 105.321705 65.103406) (end 105.926233 64.498878) (width 0.2) (layer "F.Cu") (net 23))
 (segment (start 109.731878 64.498878) (end 109.736 64.503) (width 0.2) (layer "F.Cu") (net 23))
 (segment (start 105.36783 72.83483) (end 105.36783 67.88957) (width 0.2) (layer "F.Cu") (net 18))
 (segment (start 109.736 77.203) (end 105.36783 72.83483) (width 0.2) (layer "F.Cu") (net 18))
 (segment (start 105.36783 67.88957) (end 104.756019 67.277759) (width 0.2) (layer "F.Cu") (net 18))
 (segment (start 105.604548 65.386249) (end 106.091919 64.898878) (width 0.2) (layer "F.Cu") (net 22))
 (segment (start 106.091919 64.898878) (end 107.591878 64.898878) (width 0.2) (layer "F.Cu") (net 22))
 (segment (start 107.591878 64.898878) (end 109.736 67.043) (width 0.2) (layer "F.Cu") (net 22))
 (segment (start 104.56783 63.045792) (end 104.297 62.774962) (width 0.2) (layer "F.Cu") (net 26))
 (segment (start 104.190334 63.972035) (end 104.56783 63.594539) (width 0.2) (layer "F.Cu") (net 26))
 (segment (start 104.297 62.774962) (end 104.297 59.782) (width 0.2) (layer "F.Cu") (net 26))
 (segment (start 104.297 59.782) (end 109.736 54.343) (width 0.2) (layer "F.Cu") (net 26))
 (segment (start 104.56783 63.594539) (end 104.56783 63.045792) (width 0.2) (layer "F.Cu") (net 26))
 (segment (start 105.321705 66.712074) (end 106.16783 67.558199) (width 0.2) (layer "F.Cu") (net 20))
 (segment (start 106.16783 67.558199) (end 106.16783 68.55483) (width 0.2) (layer "F.Cu") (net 20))
 (segment (start 106.16783 68.55483) (end 109.736 72.123) (width 0.2) (layer "F.Cu") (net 20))
 (segment (start 103.897 57.642) (end 109.736 51.803) (width 0.2) (layer "F.Cu") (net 27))
 (segment (start 103.897 63.678701) (end 103.897 57.642) (width 0.2) (layer "F.Cu") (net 27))
 (segment (start 103.907491 63.689192) (end 103.897 63.678701) (width 0.2) (layer "F.Cu") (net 27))
 (segment (start 105.038862 64.820563) (end 105.760547 64.098878) (width 0.2) (layer "F.Cu") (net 24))
 (segment (start 105.760547 64.098878) (end 107.600122 64.098878) (width 0.2) (layer "F.Cu") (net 24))
 (segment (start 107.600122 64.098878) (end 109.736 61.963) (width 0.2) (layer "F.Cu") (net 24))
 (segment (start 105.76783 67.723884) (end 105.76783 70.69483) (width 0.2) (layer "F.Cu") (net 19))
 (segment (start 105.038862 66.994917) (end 105.76783 67.723884) (width 0.2) (layer "F.Cu") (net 19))
 (segment (start 105.76783 70.69483) (end 109.736 74.663) (width 0.2) (layer "F.Cu") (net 19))
 (segment (start 104.473177 67.560602) (end 104.96783 68.055255) (width 0.2) (layer "F.Cu") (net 17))
 (segment (start 104.96783 68.055255) (end 104.96783 74.97483) (width 0.2) (layer "F.Cu") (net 17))
 (segment (start 104.96783 74.97483) (end 109.736 79.743) (width 0.2) (layer "F.Cu") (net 17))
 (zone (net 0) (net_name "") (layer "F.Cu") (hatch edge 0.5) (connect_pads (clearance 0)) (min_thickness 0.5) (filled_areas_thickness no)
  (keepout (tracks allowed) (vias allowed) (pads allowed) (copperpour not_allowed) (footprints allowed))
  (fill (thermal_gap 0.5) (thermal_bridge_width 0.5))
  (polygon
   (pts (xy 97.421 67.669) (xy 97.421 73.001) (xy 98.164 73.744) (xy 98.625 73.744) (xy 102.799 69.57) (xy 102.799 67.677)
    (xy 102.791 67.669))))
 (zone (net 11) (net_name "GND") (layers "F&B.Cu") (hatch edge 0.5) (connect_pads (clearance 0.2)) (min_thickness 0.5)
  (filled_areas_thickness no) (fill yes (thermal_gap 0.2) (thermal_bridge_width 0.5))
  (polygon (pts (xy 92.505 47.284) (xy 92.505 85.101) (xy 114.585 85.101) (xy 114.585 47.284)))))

